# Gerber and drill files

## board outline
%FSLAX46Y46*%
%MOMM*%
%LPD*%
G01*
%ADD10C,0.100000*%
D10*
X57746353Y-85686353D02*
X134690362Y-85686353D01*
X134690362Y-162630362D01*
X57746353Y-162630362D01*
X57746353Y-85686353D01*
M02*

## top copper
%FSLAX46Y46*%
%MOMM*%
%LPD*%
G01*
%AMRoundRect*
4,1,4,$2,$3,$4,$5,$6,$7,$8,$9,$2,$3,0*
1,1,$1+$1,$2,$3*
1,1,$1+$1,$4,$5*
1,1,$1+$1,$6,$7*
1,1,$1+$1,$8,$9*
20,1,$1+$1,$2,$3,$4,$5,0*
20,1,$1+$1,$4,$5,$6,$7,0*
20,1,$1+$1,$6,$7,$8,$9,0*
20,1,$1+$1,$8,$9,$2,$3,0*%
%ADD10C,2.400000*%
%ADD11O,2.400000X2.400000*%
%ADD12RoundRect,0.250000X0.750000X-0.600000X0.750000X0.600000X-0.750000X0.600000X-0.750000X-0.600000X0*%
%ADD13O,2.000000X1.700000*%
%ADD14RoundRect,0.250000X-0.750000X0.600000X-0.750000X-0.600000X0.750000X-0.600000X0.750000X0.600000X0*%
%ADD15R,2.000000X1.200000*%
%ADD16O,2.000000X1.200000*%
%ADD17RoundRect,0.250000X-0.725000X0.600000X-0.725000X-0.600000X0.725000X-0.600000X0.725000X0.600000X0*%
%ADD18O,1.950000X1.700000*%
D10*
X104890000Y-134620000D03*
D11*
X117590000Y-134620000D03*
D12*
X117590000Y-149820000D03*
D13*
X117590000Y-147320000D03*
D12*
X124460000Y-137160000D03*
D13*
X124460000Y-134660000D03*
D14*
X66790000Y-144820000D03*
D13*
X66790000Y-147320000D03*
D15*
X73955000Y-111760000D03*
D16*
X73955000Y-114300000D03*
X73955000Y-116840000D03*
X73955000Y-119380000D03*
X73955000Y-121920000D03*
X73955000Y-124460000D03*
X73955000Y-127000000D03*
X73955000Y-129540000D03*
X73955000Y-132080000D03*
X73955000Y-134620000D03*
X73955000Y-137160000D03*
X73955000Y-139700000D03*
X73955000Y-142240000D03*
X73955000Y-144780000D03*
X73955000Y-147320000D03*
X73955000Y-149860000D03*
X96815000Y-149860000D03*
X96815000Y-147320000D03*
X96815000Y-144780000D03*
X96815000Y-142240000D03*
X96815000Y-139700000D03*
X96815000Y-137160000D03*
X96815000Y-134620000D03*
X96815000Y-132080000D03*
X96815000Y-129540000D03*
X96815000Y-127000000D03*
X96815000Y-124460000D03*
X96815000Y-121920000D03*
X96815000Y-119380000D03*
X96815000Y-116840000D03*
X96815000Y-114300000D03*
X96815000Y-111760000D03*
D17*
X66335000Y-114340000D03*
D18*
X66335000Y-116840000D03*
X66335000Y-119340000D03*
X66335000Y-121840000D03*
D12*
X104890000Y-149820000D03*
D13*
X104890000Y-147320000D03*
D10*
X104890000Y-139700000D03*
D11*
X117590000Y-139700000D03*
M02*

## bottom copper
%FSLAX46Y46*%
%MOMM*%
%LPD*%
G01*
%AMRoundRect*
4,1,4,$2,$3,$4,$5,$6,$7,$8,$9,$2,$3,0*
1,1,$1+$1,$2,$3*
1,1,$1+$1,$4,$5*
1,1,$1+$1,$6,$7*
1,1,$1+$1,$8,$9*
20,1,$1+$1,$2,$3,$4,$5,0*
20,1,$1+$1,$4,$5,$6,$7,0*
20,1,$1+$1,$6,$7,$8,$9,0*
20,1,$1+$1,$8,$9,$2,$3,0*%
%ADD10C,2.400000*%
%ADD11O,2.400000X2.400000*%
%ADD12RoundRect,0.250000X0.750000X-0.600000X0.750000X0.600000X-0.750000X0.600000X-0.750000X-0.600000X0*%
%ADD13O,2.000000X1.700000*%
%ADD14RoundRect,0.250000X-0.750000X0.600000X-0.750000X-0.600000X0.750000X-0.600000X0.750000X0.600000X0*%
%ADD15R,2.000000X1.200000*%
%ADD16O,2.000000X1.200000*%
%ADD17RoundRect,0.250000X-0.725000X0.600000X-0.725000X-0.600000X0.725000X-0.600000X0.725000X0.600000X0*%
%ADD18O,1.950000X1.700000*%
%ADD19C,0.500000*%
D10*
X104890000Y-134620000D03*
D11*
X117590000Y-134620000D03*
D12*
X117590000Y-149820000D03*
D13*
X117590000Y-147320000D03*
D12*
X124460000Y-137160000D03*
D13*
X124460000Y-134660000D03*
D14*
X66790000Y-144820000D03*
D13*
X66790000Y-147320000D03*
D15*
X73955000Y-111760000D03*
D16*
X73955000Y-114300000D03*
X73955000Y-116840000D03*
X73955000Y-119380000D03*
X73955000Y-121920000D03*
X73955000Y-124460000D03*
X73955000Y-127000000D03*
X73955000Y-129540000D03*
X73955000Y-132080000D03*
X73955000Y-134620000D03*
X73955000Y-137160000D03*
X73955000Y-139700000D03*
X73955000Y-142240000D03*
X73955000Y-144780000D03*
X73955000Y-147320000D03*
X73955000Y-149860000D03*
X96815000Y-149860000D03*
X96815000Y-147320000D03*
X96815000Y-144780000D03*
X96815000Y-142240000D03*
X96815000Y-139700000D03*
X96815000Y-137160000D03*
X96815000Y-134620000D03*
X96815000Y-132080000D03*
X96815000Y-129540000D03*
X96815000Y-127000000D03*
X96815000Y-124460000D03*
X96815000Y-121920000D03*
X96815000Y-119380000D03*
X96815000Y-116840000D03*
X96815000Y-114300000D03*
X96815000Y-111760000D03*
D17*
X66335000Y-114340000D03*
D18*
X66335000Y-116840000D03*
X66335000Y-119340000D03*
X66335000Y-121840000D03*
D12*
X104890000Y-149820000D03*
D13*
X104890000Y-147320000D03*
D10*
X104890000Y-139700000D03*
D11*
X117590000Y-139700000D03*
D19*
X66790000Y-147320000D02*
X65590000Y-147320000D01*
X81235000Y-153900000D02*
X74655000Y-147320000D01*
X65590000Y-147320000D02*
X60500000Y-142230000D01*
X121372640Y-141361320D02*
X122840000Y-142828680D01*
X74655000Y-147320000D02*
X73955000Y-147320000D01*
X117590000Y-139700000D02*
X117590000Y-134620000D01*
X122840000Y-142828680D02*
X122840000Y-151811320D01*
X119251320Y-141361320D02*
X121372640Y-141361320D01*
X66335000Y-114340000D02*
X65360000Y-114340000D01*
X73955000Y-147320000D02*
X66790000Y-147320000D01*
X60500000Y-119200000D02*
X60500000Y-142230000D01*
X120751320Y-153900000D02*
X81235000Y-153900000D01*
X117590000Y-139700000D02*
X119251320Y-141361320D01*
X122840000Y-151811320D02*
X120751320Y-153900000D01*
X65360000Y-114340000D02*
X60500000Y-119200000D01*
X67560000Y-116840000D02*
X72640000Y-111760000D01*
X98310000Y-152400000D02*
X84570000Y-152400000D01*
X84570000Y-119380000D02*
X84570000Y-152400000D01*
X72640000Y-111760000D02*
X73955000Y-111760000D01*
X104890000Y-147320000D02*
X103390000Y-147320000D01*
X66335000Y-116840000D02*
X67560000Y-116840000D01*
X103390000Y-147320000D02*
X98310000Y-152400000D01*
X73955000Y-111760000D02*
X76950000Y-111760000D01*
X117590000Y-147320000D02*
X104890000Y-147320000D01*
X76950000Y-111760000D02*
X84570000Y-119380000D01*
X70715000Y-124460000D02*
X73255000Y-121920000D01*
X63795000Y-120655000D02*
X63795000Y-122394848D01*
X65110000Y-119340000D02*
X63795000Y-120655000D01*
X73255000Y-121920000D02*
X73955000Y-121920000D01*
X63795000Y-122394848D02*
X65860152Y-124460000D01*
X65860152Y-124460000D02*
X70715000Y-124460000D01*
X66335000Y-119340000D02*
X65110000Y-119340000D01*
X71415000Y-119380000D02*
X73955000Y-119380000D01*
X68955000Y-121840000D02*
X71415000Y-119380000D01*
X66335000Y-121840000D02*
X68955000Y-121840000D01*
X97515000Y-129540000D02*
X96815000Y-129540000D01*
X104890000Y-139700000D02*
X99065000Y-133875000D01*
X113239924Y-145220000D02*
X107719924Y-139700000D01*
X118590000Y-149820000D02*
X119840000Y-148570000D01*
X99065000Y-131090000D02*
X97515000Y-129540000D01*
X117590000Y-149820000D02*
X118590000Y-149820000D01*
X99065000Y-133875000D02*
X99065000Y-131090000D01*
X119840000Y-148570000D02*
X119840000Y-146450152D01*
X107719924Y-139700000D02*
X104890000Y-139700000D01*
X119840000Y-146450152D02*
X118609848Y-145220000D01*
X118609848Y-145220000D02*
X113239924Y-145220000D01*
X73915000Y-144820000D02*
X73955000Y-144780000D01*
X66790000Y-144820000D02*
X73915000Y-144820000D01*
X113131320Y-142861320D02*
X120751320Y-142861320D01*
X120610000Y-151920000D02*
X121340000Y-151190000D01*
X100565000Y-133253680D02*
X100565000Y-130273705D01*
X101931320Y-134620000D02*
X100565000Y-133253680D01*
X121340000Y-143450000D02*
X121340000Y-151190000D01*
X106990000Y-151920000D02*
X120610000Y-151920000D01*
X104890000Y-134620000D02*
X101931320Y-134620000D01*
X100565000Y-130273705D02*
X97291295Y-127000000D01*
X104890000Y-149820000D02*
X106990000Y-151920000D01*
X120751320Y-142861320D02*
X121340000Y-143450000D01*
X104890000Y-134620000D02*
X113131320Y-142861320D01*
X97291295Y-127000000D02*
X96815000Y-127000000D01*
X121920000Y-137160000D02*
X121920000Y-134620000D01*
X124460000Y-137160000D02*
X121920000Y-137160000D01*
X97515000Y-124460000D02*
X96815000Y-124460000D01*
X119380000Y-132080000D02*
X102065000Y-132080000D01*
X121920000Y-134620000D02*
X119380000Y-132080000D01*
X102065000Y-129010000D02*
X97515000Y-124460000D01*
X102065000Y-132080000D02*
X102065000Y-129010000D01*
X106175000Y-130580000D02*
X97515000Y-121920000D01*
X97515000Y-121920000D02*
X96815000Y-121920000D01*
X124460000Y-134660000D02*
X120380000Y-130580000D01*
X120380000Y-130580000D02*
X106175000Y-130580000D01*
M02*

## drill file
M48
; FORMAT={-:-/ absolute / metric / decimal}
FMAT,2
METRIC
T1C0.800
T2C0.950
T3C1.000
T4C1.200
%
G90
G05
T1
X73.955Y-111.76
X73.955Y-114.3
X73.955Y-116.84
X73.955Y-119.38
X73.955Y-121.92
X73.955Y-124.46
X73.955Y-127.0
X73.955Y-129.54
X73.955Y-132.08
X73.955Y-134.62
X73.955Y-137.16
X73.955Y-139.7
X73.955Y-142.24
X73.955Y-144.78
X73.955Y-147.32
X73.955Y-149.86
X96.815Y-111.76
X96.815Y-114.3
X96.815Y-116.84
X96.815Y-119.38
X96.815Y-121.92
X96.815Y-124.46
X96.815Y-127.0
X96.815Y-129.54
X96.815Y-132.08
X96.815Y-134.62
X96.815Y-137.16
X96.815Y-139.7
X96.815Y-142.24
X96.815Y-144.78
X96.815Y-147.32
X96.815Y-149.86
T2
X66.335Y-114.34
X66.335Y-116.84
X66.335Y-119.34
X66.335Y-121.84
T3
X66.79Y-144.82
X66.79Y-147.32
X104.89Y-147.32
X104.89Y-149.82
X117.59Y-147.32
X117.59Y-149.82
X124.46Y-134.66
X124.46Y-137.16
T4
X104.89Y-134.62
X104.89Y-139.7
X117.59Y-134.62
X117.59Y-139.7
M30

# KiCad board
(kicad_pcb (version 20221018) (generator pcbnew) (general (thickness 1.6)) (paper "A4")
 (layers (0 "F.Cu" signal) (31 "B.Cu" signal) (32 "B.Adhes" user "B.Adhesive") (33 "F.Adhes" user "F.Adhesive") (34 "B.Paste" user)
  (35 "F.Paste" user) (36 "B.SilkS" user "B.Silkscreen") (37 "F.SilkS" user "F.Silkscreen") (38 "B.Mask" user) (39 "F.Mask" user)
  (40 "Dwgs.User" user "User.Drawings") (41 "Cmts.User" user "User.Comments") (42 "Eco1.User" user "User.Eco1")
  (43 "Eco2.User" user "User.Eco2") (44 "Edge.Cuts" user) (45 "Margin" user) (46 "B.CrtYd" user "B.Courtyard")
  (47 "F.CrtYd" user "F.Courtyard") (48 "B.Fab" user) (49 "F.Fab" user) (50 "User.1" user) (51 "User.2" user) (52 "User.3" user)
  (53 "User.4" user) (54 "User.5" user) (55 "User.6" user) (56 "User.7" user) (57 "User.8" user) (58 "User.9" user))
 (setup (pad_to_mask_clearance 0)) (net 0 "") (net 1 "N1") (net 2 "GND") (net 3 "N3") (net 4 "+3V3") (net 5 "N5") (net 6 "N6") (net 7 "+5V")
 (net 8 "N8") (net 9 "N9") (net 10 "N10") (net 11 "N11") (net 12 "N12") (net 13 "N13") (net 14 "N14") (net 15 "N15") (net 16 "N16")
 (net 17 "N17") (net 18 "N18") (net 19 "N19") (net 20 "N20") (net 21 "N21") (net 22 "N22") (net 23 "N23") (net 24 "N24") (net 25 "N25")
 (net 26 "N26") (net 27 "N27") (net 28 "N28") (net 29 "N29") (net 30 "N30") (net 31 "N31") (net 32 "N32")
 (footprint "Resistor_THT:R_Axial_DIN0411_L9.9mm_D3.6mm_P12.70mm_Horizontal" (layer "F.Cu") (at 104.89 134.62)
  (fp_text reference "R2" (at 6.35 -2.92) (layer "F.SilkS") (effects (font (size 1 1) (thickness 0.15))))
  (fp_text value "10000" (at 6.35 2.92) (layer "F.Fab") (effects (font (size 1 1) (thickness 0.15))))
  (pad "1" thru_hole circle (at 0 0) (size 2.4 2.4) (drill 1.2) (layers "*.Cu" "*.Mask") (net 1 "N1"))
  (pad "2" thru_hole oval (at 12.7 0) (size 2.4 2.4) (drill 1.2) (layers "*.Cu" "*.Mask") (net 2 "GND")))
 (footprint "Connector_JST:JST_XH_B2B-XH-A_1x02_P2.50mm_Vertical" (layer "F.Cu") (at 117.59 149.82 90)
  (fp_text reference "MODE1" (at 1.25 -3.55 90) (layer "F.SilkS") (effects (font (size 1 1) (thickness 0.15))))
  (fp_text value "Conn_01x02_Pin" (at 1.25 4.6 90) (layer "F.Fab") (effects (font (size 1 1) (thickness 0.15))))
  (pad "1" thru_hole roundrect (at 0 0 90) (size 1.7 2) (drill 1) (layers "*.Cu" "*.Mask") (roundrect_rratio 0.1470588235) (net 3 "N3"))
  (pad "2" thru_hole oval (at 2.5 0 90) (size 1.7 2) (drill 1) (layers "*.Cu" "*.Mask") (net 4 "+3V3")))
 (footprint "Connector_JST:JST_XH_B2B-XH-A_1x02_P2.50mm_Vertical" (layer "F.Cu") (at 124.46 137.16 90)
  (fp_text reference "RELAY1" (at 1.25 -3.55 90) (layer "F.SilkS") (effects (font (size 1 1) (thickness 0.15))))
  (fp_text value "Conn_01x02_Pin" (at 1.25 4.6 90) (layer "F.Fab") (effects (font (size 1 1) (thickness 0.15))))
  (pad "1" thru_hole roundrect (at 0 0 90) (size 1.7 2) (drill 1) (layers "*.Cu" "*.Mask") (roundrect_rratio 0.1470588235) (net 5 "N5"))
  (pad "2" thru_hole oval (at 2.5 0 90) (size 1.7 2) (drill 1) (layers "*.Cu" "*.Mask") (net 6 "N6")))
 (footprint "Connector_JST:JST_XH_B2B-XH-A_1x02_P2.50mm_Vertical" (layer "F.Cu") (at 66.79 144.82 -90)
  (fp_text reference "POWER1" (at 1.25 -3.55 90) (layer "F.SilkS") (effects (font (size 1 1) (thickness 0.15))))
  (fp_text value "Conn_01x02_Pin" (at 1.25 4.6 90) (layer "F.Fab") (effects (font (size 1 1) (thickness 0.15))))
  (pad "1" thru_hole roundrect (at 0 0 270) (size 1.7 2) (drill 1) (layers "*.Cu" "*.Mask") (roundrect_rratio 0.1470588235) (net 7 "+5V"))
  (pad "2" thru_hole oval (at 2.5 0 270) (size 1.7 2) (drill 1) (layers "*.Cu" "*.Mask") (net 2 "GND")))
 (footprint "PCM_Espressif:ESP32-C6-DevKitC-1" (layer "F.Cu") (at 73.955 111.76)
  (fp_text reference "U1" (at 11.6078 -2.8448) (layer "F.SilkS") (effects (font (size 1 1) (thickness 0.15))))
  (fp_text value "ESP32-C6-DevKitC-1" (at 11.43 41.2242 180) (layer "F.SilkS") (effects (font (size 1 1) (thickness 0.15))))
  (pad "1" thru_hole rect (at 0 0 270) (size 1.2 2) (drill 0.8) (layers "*.Cu" "*.Mask") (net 4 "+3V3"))
  (pad "2" thru_hole oval (at 0 2.54 270) (size 1.2 2) (drill 0.8) (layers "*.Cu" "*.Mask") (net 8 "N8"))
  (pad "3" thru_hole oval (at 0 5.08 270) (size 1.2 2) (drill 0.8) (layers "*.Cu" "*.Mask") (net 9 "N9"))
  (pad "4" thru_hole oval (at 0 7.62 270) (size 1.2 2) (drill 0.8) (layers "*.Cu" "*.Mask") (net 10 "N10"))
  (pad "5" thru_hole oval (at 0 10.16 270) (size 1.2 2) (drill 0.8) (layers "*.Cu" "*.Mask") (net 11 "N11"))
  (pad "6" thru_hole oval (at 0 12.7 270) (size 1.2 2) (drill 0.8) (layers "*.Cu" "*.Mask") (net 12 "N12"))
  (pad "7" thru_hole oval (at 0 15.24 270) (size 1.2 2) (drill 0.8) (layers "*.Cu" "*.Mask") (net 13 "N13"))
  (pad "8" thru_hole oval (at 0 17.78 270) (size 1.2 2) (drill 0.8) (layers "*.Cu" "*.Mask") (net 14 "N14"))
  (pad "9" thru_hole oval (at 0 20.32 270) (size 1.2 2) (drill 0.8) (layers "*.Cu" "*.Mask") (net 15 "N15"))
  (pad "10" thru_hole oval (at 0 22.86 270) (size 1.2 2) (drill 0.8) (layers "*.Cu" "*.Mask") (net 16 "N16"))
  (pad "11" thru_hole oval (at 0 25.4 270) (size 1.2 2) (drill 0.8) (layers "*.Cu" "*.Mask") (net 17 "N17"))
  (pad "12" thru_hole oval (at 0 27.94 270) (size 1.2 2) (drill 0.8) (layers "*.Cu" "*.Mask") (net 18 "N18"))
  (pad "13" thru_hole oval (at 0 30.48 270) (size 1.2 2) (drill 0.8) (layers "*.Cu" "*.Mask") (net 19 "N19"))
  (pad "14" thru_hole oval (at 0 33.02 270) (size 1.2 2) (drill 0.8) (layers "*.Cu" "*.Mask") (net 7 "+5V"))
  (pad "15" thru_hole oval (at 0 35.56 270) (size 1.2 2) (drill 0.8) (layers "*.Cu" "*.Mask") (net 2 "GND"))
  (pad "16" thru_hole oval (at 0 38.1 270) (size 1.2 2) (drill 0.8) (layers "*.Cu" "*.Mask") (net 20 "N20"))
  (pad "17" thru_hole oval (at 22.86 38.1 270) (size 1.2 2) (drill 0.8) (layers "*.Cu" "*.Mask") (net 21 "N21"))
  (pad "18" thru_hole oval (at 22.86 35.56 270) (size 1.2 2) (drill 0.8) (layers "*.Cu" "*.Mask") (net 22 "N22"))
  (pad "19" thru_hole oval (at 22.86 33.02 270) (size 1.2 2) (drill 0.8) (layers "*.Cu" "*.Mask") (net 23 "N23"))
  (pad "20" thru_hole oval (at 22.86 30.48 270) (size 1.2 2) (drill 0.8) (layers "*.Cu" "*.Mask") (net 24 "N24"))
  (pad "21" thru_hole oval (at 22.86 27.94 270) (size 1.2 2) (drill 0.8) (layers "*.Cu" "*.Mask") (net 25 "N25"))
  (pad "22" thru_hole oval (at 22.86 25.4 270) (size 1.2 2) (drill 0.8) (layers "*.Cu" "*.Mask") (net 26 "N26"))
  (pad "23" thru_hole oval (at 22.86 22.86 270) (size 1.2 2) (drill 0.8) (layers "*.Cu" "*.Mask") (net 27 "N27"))
  (pad "24" thru_hole oval (at 22.86 20.32 270) (size 1.2 2) (drill 0.8) (layers "*.Cu" "*.Mask") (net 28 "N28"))
  (pad "25" thru_hole oval (at 22.86 17.78 270) (size 1.2 2) (drill 0.8) (layers "*.Cu" "*.Mask") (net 3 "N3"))
  (pad "26" thru_hole oval (at 22.86 15.24 270) (size 1.2 2) (drill 0.8) (layers "*.Cu" "*.Mask") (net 1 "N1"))
  (pad "27" thru_hole oval (at 22.86 12.7 270) (size 1.2 2) (drill 0.8) (layers "*.Cu" "*.Mask") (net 5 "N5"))
  (pad "28" thru_hole oval (at 22.86 10.16 270) (size 1.2 2) (drill 0.8) (layers "*.Cu" "*.Mask") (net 6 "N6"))
  (pad "29" thru_hole oval (at 22.86 7.62 270) (size 1.2 2) (drill 0.8) (layers "*.Cu" "*.Mask") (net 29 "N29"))
  (pad "30" thru_hole oval (at 22.86 5.08 270) (size 1.2 2) (drill 0.8) (layers "*.Cu" "*.Mask") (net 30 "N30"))
  (pad "31" thru_hole oval (at 22.86 2.54 270) (size 1.2 2) (drill 0.8) (layers "*.Cu" "*.Mask") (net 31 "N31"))
  (pad "32" thru_hole oval (at 22.86 0 270) (size 1.2 2) (drill 0.8) (layers "*.Cu" "*.Mask") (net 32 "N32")))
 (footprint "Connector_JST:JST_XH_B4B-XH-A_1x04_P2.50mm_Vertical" (layer "F.Cu") (at 66.335 114.34 -90)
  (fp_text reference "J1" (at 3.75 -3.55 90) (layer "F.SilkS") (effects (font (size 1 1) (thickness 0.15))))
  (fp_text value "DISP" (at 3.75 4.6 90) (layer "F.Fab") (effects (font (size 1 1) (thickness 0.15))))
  (pad "1" thru_hole roundrect (at 0 0 270) (size 1.7 1.95) (drill 0.95) (layers "*.Cu" "*.Mask") (roundrect_rratio 0.1470588235)
   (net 2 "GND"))
  (pad "2" thru_hole oval (at 2.5 0 270) (size 1.7 1.95) (drill 0.95) (layers "*.Cu" "*.Mask") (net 4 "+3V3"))
  (pad "3" thru_hole oval (at 5 0 270) (size 1.7 1.95) (drill 0.95) (layers "*.Cu" "*.Mask") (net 11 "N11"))
  (pad "4" thru_hole oval (at 7.5 0 270) (size 1.7 1.95) (drill 0.95) (layers "*.Cu" "*.Mask") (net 10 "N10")))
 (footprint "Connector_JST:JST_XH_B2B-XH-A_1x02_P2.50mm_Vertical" (layer "F.Cu") (at 104.89 149.82 90)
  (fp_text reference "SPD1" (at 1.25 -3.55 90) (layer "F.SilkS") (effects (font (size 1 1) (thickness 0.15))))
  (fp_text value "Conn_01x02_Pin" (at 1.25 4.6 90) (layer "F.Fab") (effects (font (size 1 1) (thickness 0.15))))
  (pad "1" thru_hole roundrect (at 0 0 90) (size 1.7 2) (drill 1) (layers "*.Cu" "*.Mask") (roundrect_rratio 0.1470588235) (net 1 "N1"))
  (pad "2" thru_hole oval (at 2.5 0 90) (size 1.7 2) (drill 1) (layers "*.Cu" "*.Mask") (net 4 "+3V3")))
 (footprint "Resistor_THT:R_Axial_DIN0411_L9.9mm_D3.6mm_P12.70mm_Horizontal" (layer "F.Cu") (at 104.89 139.7)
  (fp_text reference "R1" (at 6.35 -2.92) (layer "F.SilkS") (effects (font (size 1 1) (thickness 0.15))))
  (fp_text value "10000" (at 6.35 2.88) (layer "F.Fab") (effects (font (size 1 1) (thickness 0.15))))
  (pad "1" thru_hole circle (at 0 0) (size 2.4 2.4) (drill 1.2) (layers "*.Cu" "*.Mask") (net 3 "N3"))
  (pad "2" thru_hole oval (at 12.7 0) (size 2.4 2.4) (drill 1.2) (layers "*.Cu" "*.Mask") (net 2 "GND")))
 (gr_rect (start 57.746353 85.686353) (end 134.690362 162.630362) (stroke (width 0.1) (type default)) (fill none) (layer "Edge.Cuts"))
 (segment (start 66.79 147.32) (end 65.59 147.32) (width 0.5) (layer "B.Cu") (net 2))
 (segment (start 81.235 153.9) (end 74.655 147.32) (width 0.5) (layer "B.Cu") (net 2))
 (segment (start 65.59 147.32) (end 60.5 142.23) (width 0.5) (layer "B.Cu") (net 2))
 (segment (start 121.37264 141.36132) (end 122.84 142.82868) (width 0.5) (layer "B.Cu") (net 2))
 (segment (start 74.655 147.32) (end 73.955 147.32) (width 0.5) (layer "B.Cu") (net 2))
 (segment (start 117.59 139.7) (end 117.59 134.62) (width 0.5) (layer "B.Cu") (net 2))
 (segment (start 122.84 142.82868) (end 122.84 151.81132) (width 0.5) (layer "B.Cu") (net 2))
 (segment (start 119.25132 141.36132) (end 121.37264 141.36132) (width 0.5) (layer "B.Cu") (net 2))
 (segment (start 66.335 114.34) (end 65.36 114.34) (width 0.5) (layer "B.Cu") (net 2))
 (segment (start 73.955 147.32) (end 66.79 147.32) (width 0.5) (layer "B.Cu") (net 2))
 (segment (start 60.5 119.2) (end 60.5 142.23) (width 0.5) (layer "B.Cu") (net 2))
 (segment (start 120.75132 153.9) (end 81.235 153.9) (width 0.5) (layer "B.Cu") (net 2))
 (segment (start 117.59 139.7) (end 119.25132 141.36132) (width 0.5) (layer "B.Cu") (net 2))
 (segment (start 122.84 151.81132) (end 120.75132 153.9) (width 0.5) (layer "B.Cu") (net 2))
 (segment (start 65.36 114.34) (end 60.5 119.2) (width 0.5) (layer "B.Cu") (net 2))
 (segment (start 67.56 116.84) (end 72.64 111.76) (width 0.5) (layer "B.Cu") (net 4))
 (segment (start 98.31 152.4) (end 84.57 152.4) (width 0.5) (layer "B.Cu") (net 4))
 (segment (start 84.57 119.38) (end 84.57 152.4) (width 0.5) (layer "B.Cu") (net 4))
 (segment (start 72.64 111.76) (end 73.955 111.76) (width 0.5) (layer "B.Cu") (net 4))
 (segment (start 104.89 147.32) (end 103.39 147.32) (width 0.5) (layer "B.Cu") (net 4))
 (segment (start 66.335 116.84) (end 67.56 116.84) (width 0.5) (layer "B.Cu") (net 4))
 (segment (start 103.39 147.32) (end 98.31 152.4) (width 0.5) (layer "B.Cu") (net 4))
 (segment (start 73.955 111.76) (end 76.95 111.76) (width 0.5) (layer "B.Cu") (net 4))
 (segment (start 117.59 147.32) (end 104.89 147.32) (width 0.5) (layer "B.Cu") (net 4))
 (segment (start 76.95 111.76) (end 84.57 119.38) (width 0.5) (layer "B.Cu") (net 4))
 (segment (start 70.715 124.46) (end 73.255 121.92) (width 0.5) (layer "B.Cu") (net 11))
 (segment (start 63.795 120.655) (end 63.795 122.394848) (width 0.5) (layer "B.Cu") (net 11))
 (segment (start 65.11 119.34) (end 63.795 120.655) (width 0.5) (layer "B.Cu") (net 11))
 (segment (start 73.255 121.92) (end 73.955 121.92) (width 0.5) (layer "B.Cu") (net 11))
 (segment (start 63.795 122.394848) (end 65.860152 124.46) (width 0.5) (layer "B.Cu") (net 11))
 (segment (start 65.860152 124.46) (end 70.715 124.46) (width 0.5) (layer "B.Cu") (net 11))
 (segment (start 66.335 119.34) (end 65.11 119.34) (width 0.5) (layer "B.Cu") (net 11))
 (segment (start 71.415 119.38) (end 73.955 119.38) (width 0.5) (layer "B.Cu") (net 10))
 (segment (start 68.955 121.84) (end 71.415 119.38) (width 0.5) (layer "B.Cu") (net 10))
 (segment (start 66.335 121.84) (end 68.955 121.84) (width 0.5) (layer "B.Cu") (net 10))
 (segment (start 97.515 129.54) (end 96.815 129.54) (width 0.5) (layer "B.Cu") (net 3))
 (segment (start 104.89 139.7) (end 99.065 133.875) (width 0.5) (layer "B.Cu") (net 3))
 (segment (start 113.239924 145.22) (end 107.719924 139.7) (width 0.5) (layer "B.Cu") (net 3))
 (segment (start 118.59 149.82) (end 119.84 148.57) (width 0.5) (layer "B.Cu") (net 3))
 (segment (start 99.065 131.09) (end 97.515 129.54) (width 0.5) (layer "B.Cu") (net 3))
 (segment (start 117.59 149.82) (end 118.59 149.82) (width 0.5) (layer "B.Cu") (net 3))
 (segment (start 99.065 133.875) (end 99.065 131.09) (width 0.5) (layer "B.Cu") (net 3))
 (segment (start 119.84 148.57) (end 119.84 146.450152) (width 0.5) (layer "B.Cu") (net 3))
 (segment (start 107.719924 139.7) (end 104.89 139.7) (width 0.5) (layer "B.Cu") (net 3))
 (segment (start 119.84 146.450152) (end 118.609848 145.22) (width 0.5) (layer "B.Cu") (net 3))
 (segment (start 118.609848 145.22) (end 113.239924 145.22) (width 0.5) (layer "B.Cu") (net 3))
 (segment (start 73.915 144.82) (end 73.955 144.78) (width 0.5) (layer "B.Cu") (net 7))
 (segment (start 66.79 144.82) (end 73.915 144.82) (width 0.5) (layer "B.Cu") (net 7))
 (segment (start 113.13132 142.86132) (end 120.75132 142.86132) (width 0.5) (layer "B.Cu") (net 1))
 (segment (start 120.61 151.92) (end 121.34 151.19) (width 0.5) (layer "B.Cu") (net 1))
 (segment (start 100.565 133.25368) (end 100.565 130.273705) (width 0.5) (layer "B.Cu") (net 1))
 (segment (start 101.93132 134.62) (end 100.565 133.25368) (width 0.5) (layer "B.Cu") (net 1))
 (segment (start 121.34 143.45) (end 121.34 151.19) (width 0.5) (layer "B.Cu") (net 1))
 (segment (start 106.99 151.92) (end 120.61 151.92) (width 0.5) (layer "B.Cu") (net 1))
 (segment (start 104.89 134.62) (end 101.93132 134.62) (width 0.5) (layer "B.Cu") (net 1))
 (segment (start 100.565 130.273705) (end 97.291295 127) (width 0.5) (layer "B.Cu") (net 1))
 (segment (start 104.89 149.82) (end 106.99 151.92) (width 0.5) (layer "B.Cu") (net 1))
 (segment (start 120.75132 142.86132) (end 121.34 143.45) (width 0.5) (layer "B.Cu") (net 1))
 (segment (start 104.89 134.62) (end 113.13132 142.86132) (width 0.5) (layer "B.Cu") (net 1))
 (segment (start 97.291295 127) (end 96.815 127) (width 0.5) (layer "B.Cu") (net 1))
 (segment (start 121.92 137.16) (end 121.92 134.62) (width 0.5) (layer "B.Cu") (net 5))
 (segment (start 124.46 137.16) (end 121.92 137.16) (width 0.5) (layer "B.Cu") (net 5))
 (segment (start 97.515 124.46) (end 96.815 124.46) (width 0.5) (layer "B.Cu") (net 5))
 (segment (start 119.38 132.08) (end 102.065 132.08) (width 0.5) (layer "B.Cu") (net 5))
 (segment (start 121.92 134.62) (end 119.38 132.08) (width 0.5) (layer "B.Cu") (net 5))
 (segment (start 102.065 129.01) (end 97.515 124.46) (width 0.5) (layer "B.Cu") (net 5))
 (segment (start 102.065 132.08) (end 102.065 129.01) (width 0.5) (layer "B.Cu") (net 5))
 (segment (start 106.175 130.58) (end 97.515 121.92) (width 0.5) (layer "B.Cu") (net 6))
 (segment (start 97.515 121.92) (end 96.815 121.92) (width 0.5) (layer "B.Cu") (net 6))
 (segment (start 124.46 134.66) (end 120.38 130.58) (width 0.5) (layer "B.Cu") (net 6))
 (segment (start 120.38 130.58) (end 106.175 130.58) (width 0.5) (layer "B.Cu") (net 6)))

